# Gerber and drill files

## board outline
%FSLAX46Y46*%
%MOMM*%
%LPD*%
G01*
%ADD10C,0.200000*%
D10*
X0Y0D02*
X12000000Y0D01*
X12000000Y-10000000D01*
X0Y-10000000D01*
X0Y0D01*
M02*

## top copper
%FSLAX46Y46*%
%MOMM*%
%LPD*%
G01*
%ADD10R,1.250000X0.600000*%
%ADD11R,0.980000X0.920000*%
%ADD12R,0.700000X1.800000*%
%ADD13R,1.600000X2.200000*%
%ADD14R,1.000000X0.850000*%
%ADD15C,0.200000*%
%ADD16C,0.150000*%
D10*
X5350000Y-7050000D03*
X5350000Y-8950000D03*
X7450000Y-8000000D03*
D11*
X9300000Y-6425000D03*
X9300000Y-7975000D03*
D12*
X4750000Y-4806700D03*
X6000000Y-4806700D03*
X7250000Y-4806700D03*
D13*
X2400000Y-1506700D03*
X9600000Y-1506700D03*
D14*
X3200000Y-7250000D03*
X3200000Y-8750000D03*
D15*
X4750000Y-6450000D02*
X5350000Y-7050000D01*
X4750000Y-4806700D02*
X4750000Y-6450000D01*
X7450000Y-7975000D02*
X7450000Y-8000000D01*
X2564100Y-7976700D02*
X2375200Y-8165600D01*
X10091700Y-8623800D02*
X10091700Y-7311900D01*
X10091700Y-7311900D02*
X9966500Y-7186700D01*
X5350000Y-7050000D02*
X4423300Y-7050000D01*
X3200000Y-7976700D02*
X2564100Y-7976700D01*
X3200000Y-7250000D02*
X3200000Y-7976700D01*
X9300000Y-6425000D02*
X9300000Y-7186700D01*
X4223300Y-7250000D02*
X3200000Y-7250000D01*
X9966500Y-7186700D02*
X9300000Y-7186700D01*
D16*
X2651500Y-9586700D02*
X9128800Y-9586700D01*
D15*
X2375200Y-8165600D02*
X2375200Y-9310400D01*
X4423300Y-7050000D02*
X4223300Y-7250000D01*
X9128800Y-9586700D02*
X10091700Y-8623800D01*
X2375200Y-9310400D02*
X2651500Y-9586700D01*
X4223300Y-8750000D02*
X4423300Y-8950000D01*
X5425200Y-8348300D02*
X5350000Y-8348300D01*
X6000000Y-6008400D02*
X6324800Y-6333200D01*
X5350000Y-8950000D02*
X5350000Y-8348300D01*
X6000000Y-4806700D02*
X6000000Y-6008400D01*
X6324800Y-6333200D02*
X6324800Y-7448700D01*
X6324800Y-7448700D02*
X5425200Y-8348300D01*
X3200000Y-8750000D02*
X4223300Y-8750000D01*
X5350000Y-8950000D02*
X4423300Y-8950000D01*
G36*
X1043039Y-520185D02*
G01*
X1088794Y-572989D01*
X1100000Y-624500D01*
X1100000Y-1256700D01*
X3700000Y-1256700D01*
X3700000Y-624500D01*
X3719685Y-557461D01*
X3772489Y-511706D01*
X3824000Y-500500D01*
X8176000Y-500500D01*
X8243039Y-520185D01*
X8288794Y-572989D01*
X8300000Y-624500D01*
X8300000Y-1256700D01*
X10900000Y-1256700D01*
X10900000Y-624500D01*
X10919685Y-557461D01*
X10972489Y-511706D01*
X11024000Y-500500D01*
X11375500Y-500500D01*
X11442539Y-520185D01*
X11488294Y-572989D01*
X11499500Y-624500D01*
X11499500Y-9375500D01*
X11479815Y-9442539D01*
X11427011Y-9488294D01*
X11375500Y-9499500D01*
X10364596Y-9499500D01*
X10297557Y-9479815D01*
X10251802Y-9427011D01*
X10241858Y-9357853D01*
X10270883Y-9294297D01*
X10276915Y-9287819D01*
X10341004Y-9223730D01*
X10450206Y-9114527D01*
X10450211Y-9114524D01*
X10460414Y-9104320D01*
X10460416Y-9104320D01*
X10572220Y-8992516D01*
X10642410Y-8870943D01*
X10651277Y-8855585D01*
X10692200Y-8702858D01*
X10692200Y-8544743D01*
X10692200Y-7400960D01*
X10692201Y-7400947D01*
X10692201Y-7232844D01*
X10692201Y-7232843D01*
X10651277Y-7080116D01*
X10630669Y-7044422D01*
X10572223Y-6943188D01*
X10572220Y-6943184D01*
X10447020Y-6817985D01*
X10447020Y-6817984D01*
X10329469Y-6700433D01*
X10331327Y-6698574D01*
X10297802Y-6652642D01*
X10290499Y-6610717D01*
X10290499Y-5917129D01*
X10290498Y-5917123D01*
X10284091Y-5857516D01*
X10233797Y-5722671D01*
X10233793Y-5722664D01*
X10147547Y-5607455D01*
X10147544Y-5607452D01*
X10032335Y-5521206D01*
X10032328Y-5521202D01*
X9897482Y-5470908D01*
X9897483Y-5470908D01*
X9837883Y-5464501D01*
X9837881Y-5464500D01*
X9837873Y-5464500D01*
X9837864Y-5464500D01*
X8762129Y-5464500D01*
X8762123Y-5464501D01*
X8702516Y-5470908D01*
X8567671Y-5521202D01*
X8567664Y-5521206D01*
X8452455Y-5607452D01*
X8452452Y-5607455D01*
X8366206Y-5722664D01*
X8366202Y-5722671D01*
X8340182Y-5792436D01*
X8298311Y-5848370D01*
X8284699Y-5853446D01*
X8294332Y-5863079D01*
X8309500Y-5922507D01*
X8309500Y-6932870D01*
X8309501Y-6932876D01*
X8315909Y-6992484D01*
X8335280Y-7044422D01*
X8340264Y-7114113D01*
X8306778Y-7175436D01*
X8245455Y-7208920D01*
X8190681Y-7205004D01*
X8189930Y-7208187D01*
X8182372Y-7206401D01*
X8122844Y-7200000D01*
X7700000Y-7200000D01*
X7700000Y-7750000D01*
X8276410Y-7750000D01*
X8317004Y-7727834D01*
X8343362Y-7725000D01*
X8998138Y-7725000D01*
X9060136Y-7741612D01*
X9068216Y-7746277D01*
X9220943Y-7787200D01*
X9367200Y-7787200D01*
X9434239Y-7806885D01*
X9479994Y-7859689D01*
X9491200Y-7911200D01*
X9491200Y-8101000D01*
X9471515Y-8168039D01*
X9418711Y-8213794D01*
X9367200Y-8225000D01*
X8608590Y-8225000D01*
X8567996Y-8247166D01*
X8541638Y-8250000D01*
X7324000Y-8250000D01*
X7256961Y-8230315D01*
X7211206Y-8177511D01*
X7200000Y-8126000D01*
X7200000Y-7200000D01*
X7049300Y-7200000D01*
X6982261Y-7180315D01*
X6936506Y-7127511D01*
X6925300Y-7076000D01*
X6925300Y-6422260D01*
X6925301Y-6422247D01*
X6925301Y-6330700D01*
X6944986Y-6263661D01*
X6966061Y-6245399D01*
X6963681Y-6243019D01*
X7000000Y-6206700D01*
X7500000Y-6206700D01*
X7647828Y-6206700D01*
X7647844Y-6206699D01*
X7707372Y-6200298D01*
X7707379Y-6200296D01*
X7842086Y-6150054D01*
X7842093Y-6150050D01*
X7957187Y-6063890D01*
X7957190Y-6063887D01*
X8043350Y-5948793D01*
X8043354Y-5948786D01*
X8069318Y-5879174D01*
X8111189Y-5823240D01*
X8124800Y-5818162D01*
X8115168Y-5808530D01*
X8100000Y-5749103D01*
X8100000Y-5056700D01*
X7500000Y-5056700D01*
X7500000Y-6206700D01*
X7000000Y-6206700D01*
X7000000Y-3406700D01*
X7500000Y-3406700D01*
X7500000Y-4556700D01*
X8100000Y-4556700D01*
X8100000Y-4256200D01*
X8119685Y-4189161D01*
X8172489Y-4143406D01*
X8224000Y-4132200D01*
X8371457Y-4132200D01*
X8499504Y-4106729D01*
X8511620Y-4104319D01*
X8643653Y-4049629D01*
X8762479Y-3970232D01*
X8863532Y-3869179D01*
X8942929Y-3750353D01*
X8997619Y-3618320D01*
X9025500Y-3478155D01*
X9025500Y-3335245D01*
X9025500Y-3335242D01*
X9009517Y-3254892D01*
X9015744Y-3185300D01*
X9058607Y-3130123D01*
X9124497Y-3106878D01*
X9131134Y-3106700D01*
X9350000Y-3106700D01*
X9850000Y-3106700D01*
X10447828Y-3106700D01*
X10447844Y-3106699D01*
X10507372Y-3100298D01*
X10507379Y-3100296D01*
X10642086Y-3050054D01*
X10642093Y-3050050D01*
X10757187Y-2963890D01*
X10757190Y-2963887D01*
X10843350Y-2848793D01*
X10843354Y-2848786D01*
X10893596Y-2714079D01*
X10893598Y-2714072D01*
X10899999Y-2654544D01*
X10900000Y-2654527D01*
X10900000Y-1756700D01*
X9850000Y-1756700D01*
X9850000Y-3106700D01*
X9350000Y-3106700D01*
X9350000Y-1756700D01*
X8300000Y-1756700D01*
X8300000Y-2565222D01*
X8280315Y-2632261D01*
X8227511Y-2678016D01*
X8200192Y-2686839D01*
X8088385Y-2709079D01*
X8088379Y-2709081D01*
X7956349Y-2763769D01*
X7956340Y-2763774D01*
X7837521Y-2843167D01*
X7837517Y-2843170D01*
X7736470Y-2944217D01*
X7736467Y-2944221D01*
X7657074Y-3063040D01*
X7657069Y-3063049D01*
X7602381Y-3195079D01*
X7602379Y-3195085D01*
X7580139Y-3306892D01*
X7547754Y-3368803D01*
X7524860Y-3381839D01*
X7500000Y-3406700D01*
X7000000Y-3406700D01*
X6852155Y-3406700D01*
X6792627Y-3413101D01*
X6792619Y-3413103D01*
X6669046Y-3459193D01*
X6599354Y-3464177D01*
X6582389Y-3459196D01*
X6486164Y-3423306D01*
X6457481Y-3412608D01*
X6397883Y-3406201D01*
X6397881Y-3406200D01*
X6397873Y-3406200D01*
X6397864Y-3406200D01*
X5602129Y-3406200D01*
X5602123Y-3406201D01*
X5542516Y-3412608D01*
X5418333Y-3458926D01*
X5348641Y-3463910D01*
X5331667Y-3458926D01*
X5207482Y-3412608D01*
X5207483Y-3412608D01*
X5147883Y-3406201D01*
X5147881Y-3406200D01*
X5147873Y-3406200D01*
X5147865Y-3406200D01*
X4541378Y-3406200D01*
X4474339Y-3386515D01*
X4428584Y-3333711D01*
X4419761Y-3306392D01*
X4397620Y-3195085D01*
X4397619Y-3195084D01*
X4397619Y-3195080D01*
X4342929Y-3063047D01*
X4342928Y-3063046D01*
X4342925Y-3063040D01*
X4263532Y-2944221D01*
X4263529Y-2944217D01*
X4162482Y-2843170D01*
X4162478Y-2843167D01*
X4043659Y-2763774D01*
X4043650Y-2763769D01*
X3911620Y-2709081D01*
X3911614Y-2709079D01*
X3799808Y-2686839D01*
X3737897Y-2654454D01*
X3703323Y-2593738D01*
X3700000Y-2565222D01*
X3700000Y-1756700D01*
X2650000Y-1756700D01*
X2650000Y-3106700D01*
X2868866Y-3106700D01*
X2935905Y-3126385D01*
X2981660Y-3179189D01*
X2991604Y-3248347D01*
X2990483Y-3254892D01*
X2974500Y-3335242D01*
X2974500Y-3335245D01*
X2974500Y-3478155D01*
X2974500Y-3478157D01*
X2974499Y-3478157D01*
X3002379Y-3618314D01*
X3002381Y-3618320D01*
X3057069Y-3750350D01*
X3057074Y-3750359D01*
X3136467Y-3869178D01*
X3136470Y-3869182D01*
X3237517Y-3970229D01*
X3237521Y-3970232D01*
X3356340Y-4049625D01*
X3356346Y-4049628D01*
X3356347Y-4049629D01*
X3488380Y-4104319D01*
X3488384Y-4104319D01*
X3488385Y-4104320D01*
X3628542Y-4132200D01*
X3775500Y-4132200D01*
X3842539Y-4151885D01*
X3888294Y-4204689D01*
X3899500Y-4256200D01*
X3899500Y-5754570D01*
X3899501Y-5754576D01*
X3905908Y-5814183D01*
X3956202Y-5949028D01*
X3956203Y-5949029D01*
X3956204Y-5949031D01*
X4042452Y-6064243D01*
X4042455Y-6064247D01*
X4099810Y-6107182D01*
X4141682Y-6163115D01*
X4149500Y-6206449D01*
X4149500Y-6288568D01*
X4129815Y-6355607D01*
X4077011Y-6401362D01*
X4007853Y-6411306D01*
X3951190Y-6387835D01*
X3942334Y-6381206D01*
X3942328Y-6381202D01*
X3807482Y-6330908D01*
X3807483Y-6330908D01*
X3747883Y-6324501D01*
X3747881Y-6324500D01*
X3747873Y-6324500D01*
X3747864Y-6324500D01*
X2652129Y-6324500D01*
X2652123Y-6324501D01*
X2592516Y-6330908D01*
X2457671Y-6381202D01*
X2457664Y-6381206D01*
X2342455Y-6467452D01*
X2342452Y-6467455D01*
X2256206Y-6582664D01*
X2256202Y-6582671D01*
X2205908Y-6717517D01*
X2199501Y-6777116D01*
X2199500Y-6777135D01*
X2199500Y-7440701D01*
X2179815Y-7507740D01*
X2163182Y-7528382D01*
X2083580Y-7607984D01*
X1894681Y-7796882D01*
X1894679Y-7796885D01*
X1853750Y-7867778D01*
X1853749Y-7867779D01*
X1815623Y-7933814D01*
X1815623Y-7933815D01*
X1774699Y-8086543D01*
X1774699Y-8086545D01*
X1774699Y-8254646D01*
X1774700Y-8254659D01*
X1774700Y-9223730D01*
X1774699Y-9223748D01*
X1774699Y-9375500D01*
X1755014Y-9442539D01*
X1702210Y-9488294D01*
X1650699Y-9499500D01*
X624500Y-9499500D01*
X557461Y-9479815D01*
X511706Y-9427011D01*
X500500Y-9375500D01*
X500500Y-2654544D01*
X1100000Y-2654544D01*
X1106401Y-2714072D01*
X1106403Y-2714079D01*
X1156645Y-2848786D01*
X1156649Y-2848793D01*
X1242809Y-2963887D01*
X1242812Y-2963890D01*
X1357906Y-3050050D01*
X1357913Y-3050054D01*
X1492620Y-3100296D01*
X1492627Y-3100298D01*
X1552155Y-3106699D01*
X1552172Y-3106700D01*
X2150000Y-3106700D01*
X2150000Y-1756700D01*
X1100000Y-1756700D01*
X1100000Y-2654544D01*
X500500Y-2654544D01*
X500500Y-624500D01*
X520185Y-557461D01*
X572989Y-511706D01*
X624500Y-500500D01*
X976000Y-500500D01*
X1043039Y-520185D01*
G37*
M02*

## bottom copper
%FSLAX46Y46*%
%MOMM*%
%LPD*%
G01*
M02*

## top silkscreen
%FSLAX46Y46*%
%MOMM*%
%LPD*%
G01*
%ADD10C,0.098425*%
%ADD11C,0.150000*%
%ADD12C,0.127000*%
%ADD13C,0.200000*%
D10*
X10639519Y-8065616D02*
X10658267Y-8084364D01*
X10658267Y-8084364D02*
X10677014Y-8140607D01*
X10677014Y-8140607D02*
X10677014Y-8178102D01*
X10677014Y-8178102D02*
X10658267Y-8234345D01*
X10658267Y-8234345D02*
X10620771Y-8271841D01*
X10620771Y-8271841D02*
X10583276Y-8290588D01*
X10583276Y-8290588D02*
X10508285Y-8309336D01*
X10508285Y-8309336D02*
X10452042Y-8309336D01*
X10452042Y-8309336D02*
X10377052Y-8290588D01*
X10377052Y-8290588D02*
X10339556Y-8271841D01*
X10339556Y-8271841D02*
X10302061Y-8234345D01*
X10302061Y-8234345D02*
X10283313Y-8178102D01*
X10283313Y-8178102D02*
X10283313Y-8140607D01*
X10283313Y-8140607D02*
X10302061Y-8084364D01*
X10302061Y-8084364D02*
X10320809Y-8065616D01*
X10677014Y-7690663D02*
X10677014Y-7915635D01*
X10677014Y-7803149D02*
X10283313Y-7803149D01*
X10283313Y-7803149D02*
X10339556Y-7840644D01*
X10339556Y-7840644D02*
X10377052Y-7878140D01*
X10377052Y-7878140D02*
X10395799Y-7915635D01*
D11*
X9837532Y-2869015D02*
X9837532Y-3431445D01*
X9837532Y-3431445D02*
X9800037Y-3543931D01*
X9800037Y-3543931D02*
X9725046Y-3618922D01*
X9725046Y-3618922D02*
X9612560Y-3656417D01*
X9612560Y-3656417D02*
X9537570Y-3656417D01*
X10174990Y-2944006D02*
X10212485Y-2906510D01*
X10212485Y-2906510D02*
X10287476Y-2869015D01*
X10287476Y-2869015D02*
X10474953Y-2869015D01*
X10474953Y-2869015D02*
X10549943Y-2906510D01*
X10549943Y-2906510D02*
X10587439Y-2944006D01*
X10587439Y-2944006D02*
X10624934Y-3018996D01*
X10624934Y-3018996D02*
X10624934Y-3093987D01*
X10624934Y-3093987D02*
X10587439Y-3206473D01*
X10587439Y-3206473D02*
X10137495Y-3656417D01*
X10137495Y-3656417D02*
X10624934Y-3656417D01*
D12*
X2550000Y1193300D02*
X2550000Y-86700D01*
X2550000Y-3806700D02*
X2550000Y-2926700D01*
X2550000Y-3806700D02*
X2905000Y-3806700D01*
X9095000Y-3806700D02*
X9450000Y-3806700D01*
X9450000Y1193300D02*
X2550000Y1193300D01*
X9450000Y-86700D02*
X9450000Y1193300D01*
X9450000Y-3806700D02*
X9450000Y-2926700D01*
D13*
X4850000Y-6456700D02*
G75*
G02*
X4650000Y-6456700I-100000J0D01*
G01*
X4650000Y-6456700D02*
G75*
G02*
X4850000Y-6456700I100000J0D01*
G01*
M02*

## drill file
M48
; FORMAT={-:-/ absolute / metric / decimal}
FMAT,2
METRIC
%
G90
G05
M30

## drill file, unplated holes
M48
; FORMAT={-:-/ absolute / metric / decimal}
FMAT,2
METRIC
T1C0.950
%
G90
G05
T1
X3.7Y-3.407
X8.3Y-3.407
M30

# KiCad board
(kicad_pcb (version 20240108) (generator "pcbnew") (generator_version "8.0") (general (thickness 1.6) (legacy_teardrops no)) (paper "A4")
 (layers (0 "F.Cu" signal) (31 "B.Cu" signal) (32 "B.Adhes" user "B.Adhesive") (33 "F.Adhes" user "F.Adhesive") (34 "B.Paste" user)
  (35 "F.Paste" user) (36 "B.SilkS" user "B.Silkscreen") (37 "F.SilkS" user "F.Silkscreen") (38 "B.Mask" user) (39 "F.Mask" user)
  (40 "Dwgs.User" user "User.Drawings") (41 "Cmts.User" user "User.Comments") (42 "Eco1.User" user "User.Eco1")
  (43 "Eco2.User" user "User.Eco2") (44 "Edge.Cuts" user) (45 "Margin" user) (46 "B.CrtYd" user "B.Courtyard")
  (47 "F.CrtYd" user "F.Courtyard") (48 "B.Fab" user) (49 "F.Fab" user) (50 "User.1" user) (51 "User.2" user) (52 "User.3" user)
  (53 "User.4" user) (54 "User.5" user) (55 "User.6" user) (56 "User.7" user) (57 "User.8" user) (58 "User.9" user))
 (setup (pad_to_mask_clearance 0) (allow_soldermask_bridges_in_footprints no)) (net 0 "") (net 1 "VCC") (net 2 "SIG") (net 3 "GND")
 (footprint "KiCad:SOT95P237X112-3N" (layer "F.Cu") (at 6.4 8)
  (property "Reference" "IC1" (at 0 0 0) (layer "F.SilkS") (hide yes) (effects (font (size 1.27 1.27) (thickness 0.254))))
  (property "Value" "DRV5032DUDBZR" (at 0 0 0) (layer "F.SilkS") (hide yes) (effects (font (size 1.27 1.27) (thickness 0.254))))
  (pad "1" smd rect (at -1.05 -0.95 90) (size 0.6 1.25) (layers "F.Cu" "F.Paste" "F.Mask") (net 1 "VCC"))
  (pad "2" smd rect (at -1.05 0.95 90) (size 0.6 1.25) (layers "F.Cu" "F.Paste" "F.Mask") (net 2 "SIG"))
  (pad "3" smd rect (at 1.05 0 90) (size 0.6 1.25) (layers "F.Cu" "F.Paste" "F.Mask") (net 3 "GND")))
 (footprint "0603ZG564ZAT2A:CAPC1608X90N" (layer "F.Cu") (at 9.3 7.2 -90)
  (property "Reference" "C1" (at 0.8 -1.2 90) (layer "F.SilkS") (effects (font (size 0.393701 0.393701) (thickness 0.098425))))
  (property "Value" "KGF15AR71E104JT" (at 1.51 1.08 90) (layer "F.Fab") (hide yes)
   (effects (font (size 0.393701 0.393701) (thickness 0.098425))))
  (pad "1" smd rect (at -0.775 0 270) (size 0.92 0.98) (layers "F.Cu" "F.Paste" "F.Mask") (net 1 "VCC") (solder_mask_margin 0.102))
  (pad "2" smd rect (at 0.775 0 270) (size 0.92 0.98) (layers "F.Cu" "F.Paste" "F.Mask") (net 3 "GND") (solder_mask_margin 0.102)))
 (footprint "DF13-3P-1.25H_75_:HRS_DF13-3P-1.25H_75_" (layer "F.Cu") (at 6 3.4067)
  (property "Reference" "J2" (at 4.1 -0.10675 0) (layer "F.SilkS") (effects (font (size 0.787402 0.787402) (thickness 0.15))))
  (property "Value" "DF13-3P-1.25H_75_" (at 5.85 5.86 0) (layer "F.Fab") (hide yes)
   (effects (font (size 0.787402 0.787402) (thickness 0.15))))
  (fp_line (start -3.45 -4.6) (end -3.45 -3.32) (stroke (width 0.127) (type solid)) (layer "F.SilkS"))
  (fp_line (start -3.45 0.4) (end -3.45 -0.48) (stroke (width 0.127) (type solid)) (layer "F.SilkS"))
  (fp_line (start -3.45 0.4) (end -3.095 0.4) (stroke (width 0.127) (type solid)) (layer "F.SilkS"))
  (fp_line (start 3.095 0.4) (end 3.45 0.4) (stroke (width 0.127) (type solid)) (layer "F.SilkS"))
  (fp_line (start 3.45 -4.6) (end -3.45 -4.6) (stroke (width 0.127) (type solid)) (layer "F.SilkS"))
  (fp_line (start 3.45 -3.32) (end 3.45 -4.6) (stroke (width 0.127) (type solid)) (layer "F.SilkS"))
  (fp_line (start 3.45 0.4) (end 3.45 -0.48) (stroke (width 0.127) (type solid)) (layer "F.SilkS"))
  (fp_circle (center -1.25 3.05) (end -1.15 3.05) (stroke (width 0.2) (type solid)) (fill none) (layer "F.SilkS"))
  (pad "" np_thru_hole circle (at -2.3 0) (size 0.95 0.95) (drill 0.95) (layers "*.Cu" "*.Mask"))
  (pad "" np_thru_hole circle (at 2.3 0) (size 0.95 0.95) (drill 0.95) (layers "*.Cu" "*.Mask"))
  (pad "1" smd rect (at -1.25 1.4) (size 0.7 1.8) (layers "F.Cu" "F.Paste" "F.Mask") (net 1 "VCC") (solder_mask_margin 0.102))
  (pad "2" smd rect (at 0 1.4) (size 0.7 1.8) (layers "F.Cu" "F.Paste" "F.Mask") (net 2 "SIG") (solder_mask_margin 0.102))
  (pad "3" smd rect (at 1.25 1.4) (size 0.7 1.8) (layers "F.Cu" "F.Paste" "F.Mask") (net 3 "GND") (solder_mask_margin 0.102))
  (pad "S1" smd rect (at -3.6 -1.9) (size 1.6 2.2) (layers "F.Cu" "F.Paste" "F.Mask") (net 3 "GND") (solder_mask_margin 0.102))
  (pad "S2" smd rect (at 3.6 -1.9) (size 1.6 2.2) (layers "F.Cu" "F.Paste" "F.Mask") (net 3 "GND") (solder_mask_margin 0.102)))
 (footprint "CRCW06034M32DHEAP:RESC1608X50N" (layer "F.Cu") (at 3.2 8 -90)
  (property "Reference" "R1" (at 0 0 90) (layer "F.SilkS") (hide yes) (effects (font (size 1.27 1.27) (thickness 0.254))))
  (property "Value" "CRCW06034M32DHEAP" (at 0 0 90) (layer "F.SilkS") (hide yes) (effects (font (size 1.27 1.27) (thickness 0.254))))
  (pad "1" smd rect (at -0.75 0 270) (size 0.85 1) (layers "F.Cu" "F.Paste" "F.Mask") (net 1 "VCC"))
  (pad "2" smd rect (at 0.75 0 270) (size 0.85 1) (layers "F.Cu" "F.Paste" "F.Mask") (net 2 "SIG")))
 (gr_rect (start 0 0) (end 12 10) (stroke (width 0.2) (type default)) (fill none) (layer "Edge.Cuts"))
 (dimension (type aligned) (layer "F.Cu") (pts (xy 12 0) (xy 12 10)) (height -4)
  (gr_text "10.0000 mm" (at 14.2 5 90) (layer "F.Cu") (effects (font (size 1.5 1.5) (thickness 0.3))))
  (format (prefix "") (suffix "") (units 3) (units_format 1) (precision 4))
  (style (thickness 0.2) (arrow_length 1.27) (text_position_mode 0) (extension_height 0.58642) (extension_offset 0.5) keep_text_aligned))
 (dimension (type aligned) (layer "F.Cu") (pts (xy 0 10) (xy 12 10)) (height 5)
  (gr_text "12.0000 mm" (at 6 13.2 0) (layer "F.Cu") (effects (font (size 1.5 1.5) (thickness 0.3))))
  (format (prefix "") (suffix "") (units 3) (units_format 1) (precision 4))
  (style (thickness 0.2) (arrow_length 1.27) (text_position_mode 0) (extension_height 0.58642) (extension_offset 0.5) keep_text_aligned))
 (segment (start 7.45 7.975) (end 7.45 8) (width 0.2) (layer "F.Cu") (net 3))
 (segment (start 2.5641 7.9767) (end 2.3752 8.1656) (width 0.2) (layer "F.Cu") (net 1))
 (segment (start 10.0917 8.6238) (end 10.0917 7.3119) (width 0.2) (layer "F.Cu") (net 1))
 (segment (start 10.0917 7.3119) (end 9.9665 7.1867) (width 0.2) (layer "F.Cu") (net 1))
 (segment (start 4.75 6.45) (end 5.35 7.05) (width 0.2) (layer "F.Cu") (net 1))
 (segment (start 5.35 7.05) (end 4.4233 7.05) (width 0.2) (layer "F.Cu") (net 1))
 (segment (start 3.2 7.9767) (end 2.5641 7.9767) (width 0.2) (layer "F.Cu") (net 1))
 (segment (start 3.2 7.25) (end 3.2 7.9767) (width 0.2) (layer "F.Cu") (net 1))
 (segment (start 4.75 4.8067) (end 4.75 6.45) (width 0.2) (layer "F.Cu") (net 1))
 (segment (start 9.3 6.425) (end 9.3 7.1867) (width 0.2) (layer "F.Cu") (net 1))
 (segment (start 4.2233 7.25) (end 3.2 7.25) (width 0.2) (layer "F.Cu") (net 1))
 (segment (start 9.9665 7.1867) (end 9.3 7.1867) (width 0.2) (layer "F.Cu") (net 1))
 (segment (start 2.6515 9.5867) (end 9.1288 9.5867) (width 0.15) (layer "F.Cu") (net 1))
 (segment (start 2.3752 8.1656) (end 2.3752 9.3104) (width 0.2) (layer "F.Cu") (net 1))
 (segment (start 4.4233 7.05) (end 4.2233 7.25) (width 0.2) (layer "F.Cu") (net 1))
 (segment (start 9.1288 9.5867) (end 10.0917 8.6238) (width 0.2) (layer "F.Cu") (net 1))
 (segment (start 2.3752 9.3104) (end 2.6515 9.5867) (width 0.2) (layer "F.Cu") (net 1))
 (segment (start 4.2233 8.75) (end 4.4233 8.95) (width 0.2) (layer "F.Cu") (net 2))
 (segment (start 5.4252 8.3483) (end 5.35 8.3483) (width 0.2) (layer "F.Cu") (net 2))
 (segment (start 6 6.0084) (end 6.3248 6.3332) (width 0.2) (layer "F.Cu") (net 2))
 (segment (start 5.35 8.95) (end 5.35 8.3483) (width 0.2) (layer "F.Cu") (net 2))
 (segment (start 6 4.8067) (end 6 6.0084) (width 0.2) (layer "F.Cu") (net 2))
 (segment (start 6.3248 6.3332) (end 6.3248 7.4487) (width 0.2) (layer "F.Cu") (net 2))
 (segment (start 6.3248 7.4487) (end 5.4252 8.3483) (width 0.2) (layer "F.Cu") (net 2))
 (segment (start 3.2 8.75) (end 4.2233 8.75) (width 0.2) (layer "F.Cu") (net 2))
 (segment (start 5.35 8.95) (end 4.4233 8.95) (width 0.2) (layer "F.Cu") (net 2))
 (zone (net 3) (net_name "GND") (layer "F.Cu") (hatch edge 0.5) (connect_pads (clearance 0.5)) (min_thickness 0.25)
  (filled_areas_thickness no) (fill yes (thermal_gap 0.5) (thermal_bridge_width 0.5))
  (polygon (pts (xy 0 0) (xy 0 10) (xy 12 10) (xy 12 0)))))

